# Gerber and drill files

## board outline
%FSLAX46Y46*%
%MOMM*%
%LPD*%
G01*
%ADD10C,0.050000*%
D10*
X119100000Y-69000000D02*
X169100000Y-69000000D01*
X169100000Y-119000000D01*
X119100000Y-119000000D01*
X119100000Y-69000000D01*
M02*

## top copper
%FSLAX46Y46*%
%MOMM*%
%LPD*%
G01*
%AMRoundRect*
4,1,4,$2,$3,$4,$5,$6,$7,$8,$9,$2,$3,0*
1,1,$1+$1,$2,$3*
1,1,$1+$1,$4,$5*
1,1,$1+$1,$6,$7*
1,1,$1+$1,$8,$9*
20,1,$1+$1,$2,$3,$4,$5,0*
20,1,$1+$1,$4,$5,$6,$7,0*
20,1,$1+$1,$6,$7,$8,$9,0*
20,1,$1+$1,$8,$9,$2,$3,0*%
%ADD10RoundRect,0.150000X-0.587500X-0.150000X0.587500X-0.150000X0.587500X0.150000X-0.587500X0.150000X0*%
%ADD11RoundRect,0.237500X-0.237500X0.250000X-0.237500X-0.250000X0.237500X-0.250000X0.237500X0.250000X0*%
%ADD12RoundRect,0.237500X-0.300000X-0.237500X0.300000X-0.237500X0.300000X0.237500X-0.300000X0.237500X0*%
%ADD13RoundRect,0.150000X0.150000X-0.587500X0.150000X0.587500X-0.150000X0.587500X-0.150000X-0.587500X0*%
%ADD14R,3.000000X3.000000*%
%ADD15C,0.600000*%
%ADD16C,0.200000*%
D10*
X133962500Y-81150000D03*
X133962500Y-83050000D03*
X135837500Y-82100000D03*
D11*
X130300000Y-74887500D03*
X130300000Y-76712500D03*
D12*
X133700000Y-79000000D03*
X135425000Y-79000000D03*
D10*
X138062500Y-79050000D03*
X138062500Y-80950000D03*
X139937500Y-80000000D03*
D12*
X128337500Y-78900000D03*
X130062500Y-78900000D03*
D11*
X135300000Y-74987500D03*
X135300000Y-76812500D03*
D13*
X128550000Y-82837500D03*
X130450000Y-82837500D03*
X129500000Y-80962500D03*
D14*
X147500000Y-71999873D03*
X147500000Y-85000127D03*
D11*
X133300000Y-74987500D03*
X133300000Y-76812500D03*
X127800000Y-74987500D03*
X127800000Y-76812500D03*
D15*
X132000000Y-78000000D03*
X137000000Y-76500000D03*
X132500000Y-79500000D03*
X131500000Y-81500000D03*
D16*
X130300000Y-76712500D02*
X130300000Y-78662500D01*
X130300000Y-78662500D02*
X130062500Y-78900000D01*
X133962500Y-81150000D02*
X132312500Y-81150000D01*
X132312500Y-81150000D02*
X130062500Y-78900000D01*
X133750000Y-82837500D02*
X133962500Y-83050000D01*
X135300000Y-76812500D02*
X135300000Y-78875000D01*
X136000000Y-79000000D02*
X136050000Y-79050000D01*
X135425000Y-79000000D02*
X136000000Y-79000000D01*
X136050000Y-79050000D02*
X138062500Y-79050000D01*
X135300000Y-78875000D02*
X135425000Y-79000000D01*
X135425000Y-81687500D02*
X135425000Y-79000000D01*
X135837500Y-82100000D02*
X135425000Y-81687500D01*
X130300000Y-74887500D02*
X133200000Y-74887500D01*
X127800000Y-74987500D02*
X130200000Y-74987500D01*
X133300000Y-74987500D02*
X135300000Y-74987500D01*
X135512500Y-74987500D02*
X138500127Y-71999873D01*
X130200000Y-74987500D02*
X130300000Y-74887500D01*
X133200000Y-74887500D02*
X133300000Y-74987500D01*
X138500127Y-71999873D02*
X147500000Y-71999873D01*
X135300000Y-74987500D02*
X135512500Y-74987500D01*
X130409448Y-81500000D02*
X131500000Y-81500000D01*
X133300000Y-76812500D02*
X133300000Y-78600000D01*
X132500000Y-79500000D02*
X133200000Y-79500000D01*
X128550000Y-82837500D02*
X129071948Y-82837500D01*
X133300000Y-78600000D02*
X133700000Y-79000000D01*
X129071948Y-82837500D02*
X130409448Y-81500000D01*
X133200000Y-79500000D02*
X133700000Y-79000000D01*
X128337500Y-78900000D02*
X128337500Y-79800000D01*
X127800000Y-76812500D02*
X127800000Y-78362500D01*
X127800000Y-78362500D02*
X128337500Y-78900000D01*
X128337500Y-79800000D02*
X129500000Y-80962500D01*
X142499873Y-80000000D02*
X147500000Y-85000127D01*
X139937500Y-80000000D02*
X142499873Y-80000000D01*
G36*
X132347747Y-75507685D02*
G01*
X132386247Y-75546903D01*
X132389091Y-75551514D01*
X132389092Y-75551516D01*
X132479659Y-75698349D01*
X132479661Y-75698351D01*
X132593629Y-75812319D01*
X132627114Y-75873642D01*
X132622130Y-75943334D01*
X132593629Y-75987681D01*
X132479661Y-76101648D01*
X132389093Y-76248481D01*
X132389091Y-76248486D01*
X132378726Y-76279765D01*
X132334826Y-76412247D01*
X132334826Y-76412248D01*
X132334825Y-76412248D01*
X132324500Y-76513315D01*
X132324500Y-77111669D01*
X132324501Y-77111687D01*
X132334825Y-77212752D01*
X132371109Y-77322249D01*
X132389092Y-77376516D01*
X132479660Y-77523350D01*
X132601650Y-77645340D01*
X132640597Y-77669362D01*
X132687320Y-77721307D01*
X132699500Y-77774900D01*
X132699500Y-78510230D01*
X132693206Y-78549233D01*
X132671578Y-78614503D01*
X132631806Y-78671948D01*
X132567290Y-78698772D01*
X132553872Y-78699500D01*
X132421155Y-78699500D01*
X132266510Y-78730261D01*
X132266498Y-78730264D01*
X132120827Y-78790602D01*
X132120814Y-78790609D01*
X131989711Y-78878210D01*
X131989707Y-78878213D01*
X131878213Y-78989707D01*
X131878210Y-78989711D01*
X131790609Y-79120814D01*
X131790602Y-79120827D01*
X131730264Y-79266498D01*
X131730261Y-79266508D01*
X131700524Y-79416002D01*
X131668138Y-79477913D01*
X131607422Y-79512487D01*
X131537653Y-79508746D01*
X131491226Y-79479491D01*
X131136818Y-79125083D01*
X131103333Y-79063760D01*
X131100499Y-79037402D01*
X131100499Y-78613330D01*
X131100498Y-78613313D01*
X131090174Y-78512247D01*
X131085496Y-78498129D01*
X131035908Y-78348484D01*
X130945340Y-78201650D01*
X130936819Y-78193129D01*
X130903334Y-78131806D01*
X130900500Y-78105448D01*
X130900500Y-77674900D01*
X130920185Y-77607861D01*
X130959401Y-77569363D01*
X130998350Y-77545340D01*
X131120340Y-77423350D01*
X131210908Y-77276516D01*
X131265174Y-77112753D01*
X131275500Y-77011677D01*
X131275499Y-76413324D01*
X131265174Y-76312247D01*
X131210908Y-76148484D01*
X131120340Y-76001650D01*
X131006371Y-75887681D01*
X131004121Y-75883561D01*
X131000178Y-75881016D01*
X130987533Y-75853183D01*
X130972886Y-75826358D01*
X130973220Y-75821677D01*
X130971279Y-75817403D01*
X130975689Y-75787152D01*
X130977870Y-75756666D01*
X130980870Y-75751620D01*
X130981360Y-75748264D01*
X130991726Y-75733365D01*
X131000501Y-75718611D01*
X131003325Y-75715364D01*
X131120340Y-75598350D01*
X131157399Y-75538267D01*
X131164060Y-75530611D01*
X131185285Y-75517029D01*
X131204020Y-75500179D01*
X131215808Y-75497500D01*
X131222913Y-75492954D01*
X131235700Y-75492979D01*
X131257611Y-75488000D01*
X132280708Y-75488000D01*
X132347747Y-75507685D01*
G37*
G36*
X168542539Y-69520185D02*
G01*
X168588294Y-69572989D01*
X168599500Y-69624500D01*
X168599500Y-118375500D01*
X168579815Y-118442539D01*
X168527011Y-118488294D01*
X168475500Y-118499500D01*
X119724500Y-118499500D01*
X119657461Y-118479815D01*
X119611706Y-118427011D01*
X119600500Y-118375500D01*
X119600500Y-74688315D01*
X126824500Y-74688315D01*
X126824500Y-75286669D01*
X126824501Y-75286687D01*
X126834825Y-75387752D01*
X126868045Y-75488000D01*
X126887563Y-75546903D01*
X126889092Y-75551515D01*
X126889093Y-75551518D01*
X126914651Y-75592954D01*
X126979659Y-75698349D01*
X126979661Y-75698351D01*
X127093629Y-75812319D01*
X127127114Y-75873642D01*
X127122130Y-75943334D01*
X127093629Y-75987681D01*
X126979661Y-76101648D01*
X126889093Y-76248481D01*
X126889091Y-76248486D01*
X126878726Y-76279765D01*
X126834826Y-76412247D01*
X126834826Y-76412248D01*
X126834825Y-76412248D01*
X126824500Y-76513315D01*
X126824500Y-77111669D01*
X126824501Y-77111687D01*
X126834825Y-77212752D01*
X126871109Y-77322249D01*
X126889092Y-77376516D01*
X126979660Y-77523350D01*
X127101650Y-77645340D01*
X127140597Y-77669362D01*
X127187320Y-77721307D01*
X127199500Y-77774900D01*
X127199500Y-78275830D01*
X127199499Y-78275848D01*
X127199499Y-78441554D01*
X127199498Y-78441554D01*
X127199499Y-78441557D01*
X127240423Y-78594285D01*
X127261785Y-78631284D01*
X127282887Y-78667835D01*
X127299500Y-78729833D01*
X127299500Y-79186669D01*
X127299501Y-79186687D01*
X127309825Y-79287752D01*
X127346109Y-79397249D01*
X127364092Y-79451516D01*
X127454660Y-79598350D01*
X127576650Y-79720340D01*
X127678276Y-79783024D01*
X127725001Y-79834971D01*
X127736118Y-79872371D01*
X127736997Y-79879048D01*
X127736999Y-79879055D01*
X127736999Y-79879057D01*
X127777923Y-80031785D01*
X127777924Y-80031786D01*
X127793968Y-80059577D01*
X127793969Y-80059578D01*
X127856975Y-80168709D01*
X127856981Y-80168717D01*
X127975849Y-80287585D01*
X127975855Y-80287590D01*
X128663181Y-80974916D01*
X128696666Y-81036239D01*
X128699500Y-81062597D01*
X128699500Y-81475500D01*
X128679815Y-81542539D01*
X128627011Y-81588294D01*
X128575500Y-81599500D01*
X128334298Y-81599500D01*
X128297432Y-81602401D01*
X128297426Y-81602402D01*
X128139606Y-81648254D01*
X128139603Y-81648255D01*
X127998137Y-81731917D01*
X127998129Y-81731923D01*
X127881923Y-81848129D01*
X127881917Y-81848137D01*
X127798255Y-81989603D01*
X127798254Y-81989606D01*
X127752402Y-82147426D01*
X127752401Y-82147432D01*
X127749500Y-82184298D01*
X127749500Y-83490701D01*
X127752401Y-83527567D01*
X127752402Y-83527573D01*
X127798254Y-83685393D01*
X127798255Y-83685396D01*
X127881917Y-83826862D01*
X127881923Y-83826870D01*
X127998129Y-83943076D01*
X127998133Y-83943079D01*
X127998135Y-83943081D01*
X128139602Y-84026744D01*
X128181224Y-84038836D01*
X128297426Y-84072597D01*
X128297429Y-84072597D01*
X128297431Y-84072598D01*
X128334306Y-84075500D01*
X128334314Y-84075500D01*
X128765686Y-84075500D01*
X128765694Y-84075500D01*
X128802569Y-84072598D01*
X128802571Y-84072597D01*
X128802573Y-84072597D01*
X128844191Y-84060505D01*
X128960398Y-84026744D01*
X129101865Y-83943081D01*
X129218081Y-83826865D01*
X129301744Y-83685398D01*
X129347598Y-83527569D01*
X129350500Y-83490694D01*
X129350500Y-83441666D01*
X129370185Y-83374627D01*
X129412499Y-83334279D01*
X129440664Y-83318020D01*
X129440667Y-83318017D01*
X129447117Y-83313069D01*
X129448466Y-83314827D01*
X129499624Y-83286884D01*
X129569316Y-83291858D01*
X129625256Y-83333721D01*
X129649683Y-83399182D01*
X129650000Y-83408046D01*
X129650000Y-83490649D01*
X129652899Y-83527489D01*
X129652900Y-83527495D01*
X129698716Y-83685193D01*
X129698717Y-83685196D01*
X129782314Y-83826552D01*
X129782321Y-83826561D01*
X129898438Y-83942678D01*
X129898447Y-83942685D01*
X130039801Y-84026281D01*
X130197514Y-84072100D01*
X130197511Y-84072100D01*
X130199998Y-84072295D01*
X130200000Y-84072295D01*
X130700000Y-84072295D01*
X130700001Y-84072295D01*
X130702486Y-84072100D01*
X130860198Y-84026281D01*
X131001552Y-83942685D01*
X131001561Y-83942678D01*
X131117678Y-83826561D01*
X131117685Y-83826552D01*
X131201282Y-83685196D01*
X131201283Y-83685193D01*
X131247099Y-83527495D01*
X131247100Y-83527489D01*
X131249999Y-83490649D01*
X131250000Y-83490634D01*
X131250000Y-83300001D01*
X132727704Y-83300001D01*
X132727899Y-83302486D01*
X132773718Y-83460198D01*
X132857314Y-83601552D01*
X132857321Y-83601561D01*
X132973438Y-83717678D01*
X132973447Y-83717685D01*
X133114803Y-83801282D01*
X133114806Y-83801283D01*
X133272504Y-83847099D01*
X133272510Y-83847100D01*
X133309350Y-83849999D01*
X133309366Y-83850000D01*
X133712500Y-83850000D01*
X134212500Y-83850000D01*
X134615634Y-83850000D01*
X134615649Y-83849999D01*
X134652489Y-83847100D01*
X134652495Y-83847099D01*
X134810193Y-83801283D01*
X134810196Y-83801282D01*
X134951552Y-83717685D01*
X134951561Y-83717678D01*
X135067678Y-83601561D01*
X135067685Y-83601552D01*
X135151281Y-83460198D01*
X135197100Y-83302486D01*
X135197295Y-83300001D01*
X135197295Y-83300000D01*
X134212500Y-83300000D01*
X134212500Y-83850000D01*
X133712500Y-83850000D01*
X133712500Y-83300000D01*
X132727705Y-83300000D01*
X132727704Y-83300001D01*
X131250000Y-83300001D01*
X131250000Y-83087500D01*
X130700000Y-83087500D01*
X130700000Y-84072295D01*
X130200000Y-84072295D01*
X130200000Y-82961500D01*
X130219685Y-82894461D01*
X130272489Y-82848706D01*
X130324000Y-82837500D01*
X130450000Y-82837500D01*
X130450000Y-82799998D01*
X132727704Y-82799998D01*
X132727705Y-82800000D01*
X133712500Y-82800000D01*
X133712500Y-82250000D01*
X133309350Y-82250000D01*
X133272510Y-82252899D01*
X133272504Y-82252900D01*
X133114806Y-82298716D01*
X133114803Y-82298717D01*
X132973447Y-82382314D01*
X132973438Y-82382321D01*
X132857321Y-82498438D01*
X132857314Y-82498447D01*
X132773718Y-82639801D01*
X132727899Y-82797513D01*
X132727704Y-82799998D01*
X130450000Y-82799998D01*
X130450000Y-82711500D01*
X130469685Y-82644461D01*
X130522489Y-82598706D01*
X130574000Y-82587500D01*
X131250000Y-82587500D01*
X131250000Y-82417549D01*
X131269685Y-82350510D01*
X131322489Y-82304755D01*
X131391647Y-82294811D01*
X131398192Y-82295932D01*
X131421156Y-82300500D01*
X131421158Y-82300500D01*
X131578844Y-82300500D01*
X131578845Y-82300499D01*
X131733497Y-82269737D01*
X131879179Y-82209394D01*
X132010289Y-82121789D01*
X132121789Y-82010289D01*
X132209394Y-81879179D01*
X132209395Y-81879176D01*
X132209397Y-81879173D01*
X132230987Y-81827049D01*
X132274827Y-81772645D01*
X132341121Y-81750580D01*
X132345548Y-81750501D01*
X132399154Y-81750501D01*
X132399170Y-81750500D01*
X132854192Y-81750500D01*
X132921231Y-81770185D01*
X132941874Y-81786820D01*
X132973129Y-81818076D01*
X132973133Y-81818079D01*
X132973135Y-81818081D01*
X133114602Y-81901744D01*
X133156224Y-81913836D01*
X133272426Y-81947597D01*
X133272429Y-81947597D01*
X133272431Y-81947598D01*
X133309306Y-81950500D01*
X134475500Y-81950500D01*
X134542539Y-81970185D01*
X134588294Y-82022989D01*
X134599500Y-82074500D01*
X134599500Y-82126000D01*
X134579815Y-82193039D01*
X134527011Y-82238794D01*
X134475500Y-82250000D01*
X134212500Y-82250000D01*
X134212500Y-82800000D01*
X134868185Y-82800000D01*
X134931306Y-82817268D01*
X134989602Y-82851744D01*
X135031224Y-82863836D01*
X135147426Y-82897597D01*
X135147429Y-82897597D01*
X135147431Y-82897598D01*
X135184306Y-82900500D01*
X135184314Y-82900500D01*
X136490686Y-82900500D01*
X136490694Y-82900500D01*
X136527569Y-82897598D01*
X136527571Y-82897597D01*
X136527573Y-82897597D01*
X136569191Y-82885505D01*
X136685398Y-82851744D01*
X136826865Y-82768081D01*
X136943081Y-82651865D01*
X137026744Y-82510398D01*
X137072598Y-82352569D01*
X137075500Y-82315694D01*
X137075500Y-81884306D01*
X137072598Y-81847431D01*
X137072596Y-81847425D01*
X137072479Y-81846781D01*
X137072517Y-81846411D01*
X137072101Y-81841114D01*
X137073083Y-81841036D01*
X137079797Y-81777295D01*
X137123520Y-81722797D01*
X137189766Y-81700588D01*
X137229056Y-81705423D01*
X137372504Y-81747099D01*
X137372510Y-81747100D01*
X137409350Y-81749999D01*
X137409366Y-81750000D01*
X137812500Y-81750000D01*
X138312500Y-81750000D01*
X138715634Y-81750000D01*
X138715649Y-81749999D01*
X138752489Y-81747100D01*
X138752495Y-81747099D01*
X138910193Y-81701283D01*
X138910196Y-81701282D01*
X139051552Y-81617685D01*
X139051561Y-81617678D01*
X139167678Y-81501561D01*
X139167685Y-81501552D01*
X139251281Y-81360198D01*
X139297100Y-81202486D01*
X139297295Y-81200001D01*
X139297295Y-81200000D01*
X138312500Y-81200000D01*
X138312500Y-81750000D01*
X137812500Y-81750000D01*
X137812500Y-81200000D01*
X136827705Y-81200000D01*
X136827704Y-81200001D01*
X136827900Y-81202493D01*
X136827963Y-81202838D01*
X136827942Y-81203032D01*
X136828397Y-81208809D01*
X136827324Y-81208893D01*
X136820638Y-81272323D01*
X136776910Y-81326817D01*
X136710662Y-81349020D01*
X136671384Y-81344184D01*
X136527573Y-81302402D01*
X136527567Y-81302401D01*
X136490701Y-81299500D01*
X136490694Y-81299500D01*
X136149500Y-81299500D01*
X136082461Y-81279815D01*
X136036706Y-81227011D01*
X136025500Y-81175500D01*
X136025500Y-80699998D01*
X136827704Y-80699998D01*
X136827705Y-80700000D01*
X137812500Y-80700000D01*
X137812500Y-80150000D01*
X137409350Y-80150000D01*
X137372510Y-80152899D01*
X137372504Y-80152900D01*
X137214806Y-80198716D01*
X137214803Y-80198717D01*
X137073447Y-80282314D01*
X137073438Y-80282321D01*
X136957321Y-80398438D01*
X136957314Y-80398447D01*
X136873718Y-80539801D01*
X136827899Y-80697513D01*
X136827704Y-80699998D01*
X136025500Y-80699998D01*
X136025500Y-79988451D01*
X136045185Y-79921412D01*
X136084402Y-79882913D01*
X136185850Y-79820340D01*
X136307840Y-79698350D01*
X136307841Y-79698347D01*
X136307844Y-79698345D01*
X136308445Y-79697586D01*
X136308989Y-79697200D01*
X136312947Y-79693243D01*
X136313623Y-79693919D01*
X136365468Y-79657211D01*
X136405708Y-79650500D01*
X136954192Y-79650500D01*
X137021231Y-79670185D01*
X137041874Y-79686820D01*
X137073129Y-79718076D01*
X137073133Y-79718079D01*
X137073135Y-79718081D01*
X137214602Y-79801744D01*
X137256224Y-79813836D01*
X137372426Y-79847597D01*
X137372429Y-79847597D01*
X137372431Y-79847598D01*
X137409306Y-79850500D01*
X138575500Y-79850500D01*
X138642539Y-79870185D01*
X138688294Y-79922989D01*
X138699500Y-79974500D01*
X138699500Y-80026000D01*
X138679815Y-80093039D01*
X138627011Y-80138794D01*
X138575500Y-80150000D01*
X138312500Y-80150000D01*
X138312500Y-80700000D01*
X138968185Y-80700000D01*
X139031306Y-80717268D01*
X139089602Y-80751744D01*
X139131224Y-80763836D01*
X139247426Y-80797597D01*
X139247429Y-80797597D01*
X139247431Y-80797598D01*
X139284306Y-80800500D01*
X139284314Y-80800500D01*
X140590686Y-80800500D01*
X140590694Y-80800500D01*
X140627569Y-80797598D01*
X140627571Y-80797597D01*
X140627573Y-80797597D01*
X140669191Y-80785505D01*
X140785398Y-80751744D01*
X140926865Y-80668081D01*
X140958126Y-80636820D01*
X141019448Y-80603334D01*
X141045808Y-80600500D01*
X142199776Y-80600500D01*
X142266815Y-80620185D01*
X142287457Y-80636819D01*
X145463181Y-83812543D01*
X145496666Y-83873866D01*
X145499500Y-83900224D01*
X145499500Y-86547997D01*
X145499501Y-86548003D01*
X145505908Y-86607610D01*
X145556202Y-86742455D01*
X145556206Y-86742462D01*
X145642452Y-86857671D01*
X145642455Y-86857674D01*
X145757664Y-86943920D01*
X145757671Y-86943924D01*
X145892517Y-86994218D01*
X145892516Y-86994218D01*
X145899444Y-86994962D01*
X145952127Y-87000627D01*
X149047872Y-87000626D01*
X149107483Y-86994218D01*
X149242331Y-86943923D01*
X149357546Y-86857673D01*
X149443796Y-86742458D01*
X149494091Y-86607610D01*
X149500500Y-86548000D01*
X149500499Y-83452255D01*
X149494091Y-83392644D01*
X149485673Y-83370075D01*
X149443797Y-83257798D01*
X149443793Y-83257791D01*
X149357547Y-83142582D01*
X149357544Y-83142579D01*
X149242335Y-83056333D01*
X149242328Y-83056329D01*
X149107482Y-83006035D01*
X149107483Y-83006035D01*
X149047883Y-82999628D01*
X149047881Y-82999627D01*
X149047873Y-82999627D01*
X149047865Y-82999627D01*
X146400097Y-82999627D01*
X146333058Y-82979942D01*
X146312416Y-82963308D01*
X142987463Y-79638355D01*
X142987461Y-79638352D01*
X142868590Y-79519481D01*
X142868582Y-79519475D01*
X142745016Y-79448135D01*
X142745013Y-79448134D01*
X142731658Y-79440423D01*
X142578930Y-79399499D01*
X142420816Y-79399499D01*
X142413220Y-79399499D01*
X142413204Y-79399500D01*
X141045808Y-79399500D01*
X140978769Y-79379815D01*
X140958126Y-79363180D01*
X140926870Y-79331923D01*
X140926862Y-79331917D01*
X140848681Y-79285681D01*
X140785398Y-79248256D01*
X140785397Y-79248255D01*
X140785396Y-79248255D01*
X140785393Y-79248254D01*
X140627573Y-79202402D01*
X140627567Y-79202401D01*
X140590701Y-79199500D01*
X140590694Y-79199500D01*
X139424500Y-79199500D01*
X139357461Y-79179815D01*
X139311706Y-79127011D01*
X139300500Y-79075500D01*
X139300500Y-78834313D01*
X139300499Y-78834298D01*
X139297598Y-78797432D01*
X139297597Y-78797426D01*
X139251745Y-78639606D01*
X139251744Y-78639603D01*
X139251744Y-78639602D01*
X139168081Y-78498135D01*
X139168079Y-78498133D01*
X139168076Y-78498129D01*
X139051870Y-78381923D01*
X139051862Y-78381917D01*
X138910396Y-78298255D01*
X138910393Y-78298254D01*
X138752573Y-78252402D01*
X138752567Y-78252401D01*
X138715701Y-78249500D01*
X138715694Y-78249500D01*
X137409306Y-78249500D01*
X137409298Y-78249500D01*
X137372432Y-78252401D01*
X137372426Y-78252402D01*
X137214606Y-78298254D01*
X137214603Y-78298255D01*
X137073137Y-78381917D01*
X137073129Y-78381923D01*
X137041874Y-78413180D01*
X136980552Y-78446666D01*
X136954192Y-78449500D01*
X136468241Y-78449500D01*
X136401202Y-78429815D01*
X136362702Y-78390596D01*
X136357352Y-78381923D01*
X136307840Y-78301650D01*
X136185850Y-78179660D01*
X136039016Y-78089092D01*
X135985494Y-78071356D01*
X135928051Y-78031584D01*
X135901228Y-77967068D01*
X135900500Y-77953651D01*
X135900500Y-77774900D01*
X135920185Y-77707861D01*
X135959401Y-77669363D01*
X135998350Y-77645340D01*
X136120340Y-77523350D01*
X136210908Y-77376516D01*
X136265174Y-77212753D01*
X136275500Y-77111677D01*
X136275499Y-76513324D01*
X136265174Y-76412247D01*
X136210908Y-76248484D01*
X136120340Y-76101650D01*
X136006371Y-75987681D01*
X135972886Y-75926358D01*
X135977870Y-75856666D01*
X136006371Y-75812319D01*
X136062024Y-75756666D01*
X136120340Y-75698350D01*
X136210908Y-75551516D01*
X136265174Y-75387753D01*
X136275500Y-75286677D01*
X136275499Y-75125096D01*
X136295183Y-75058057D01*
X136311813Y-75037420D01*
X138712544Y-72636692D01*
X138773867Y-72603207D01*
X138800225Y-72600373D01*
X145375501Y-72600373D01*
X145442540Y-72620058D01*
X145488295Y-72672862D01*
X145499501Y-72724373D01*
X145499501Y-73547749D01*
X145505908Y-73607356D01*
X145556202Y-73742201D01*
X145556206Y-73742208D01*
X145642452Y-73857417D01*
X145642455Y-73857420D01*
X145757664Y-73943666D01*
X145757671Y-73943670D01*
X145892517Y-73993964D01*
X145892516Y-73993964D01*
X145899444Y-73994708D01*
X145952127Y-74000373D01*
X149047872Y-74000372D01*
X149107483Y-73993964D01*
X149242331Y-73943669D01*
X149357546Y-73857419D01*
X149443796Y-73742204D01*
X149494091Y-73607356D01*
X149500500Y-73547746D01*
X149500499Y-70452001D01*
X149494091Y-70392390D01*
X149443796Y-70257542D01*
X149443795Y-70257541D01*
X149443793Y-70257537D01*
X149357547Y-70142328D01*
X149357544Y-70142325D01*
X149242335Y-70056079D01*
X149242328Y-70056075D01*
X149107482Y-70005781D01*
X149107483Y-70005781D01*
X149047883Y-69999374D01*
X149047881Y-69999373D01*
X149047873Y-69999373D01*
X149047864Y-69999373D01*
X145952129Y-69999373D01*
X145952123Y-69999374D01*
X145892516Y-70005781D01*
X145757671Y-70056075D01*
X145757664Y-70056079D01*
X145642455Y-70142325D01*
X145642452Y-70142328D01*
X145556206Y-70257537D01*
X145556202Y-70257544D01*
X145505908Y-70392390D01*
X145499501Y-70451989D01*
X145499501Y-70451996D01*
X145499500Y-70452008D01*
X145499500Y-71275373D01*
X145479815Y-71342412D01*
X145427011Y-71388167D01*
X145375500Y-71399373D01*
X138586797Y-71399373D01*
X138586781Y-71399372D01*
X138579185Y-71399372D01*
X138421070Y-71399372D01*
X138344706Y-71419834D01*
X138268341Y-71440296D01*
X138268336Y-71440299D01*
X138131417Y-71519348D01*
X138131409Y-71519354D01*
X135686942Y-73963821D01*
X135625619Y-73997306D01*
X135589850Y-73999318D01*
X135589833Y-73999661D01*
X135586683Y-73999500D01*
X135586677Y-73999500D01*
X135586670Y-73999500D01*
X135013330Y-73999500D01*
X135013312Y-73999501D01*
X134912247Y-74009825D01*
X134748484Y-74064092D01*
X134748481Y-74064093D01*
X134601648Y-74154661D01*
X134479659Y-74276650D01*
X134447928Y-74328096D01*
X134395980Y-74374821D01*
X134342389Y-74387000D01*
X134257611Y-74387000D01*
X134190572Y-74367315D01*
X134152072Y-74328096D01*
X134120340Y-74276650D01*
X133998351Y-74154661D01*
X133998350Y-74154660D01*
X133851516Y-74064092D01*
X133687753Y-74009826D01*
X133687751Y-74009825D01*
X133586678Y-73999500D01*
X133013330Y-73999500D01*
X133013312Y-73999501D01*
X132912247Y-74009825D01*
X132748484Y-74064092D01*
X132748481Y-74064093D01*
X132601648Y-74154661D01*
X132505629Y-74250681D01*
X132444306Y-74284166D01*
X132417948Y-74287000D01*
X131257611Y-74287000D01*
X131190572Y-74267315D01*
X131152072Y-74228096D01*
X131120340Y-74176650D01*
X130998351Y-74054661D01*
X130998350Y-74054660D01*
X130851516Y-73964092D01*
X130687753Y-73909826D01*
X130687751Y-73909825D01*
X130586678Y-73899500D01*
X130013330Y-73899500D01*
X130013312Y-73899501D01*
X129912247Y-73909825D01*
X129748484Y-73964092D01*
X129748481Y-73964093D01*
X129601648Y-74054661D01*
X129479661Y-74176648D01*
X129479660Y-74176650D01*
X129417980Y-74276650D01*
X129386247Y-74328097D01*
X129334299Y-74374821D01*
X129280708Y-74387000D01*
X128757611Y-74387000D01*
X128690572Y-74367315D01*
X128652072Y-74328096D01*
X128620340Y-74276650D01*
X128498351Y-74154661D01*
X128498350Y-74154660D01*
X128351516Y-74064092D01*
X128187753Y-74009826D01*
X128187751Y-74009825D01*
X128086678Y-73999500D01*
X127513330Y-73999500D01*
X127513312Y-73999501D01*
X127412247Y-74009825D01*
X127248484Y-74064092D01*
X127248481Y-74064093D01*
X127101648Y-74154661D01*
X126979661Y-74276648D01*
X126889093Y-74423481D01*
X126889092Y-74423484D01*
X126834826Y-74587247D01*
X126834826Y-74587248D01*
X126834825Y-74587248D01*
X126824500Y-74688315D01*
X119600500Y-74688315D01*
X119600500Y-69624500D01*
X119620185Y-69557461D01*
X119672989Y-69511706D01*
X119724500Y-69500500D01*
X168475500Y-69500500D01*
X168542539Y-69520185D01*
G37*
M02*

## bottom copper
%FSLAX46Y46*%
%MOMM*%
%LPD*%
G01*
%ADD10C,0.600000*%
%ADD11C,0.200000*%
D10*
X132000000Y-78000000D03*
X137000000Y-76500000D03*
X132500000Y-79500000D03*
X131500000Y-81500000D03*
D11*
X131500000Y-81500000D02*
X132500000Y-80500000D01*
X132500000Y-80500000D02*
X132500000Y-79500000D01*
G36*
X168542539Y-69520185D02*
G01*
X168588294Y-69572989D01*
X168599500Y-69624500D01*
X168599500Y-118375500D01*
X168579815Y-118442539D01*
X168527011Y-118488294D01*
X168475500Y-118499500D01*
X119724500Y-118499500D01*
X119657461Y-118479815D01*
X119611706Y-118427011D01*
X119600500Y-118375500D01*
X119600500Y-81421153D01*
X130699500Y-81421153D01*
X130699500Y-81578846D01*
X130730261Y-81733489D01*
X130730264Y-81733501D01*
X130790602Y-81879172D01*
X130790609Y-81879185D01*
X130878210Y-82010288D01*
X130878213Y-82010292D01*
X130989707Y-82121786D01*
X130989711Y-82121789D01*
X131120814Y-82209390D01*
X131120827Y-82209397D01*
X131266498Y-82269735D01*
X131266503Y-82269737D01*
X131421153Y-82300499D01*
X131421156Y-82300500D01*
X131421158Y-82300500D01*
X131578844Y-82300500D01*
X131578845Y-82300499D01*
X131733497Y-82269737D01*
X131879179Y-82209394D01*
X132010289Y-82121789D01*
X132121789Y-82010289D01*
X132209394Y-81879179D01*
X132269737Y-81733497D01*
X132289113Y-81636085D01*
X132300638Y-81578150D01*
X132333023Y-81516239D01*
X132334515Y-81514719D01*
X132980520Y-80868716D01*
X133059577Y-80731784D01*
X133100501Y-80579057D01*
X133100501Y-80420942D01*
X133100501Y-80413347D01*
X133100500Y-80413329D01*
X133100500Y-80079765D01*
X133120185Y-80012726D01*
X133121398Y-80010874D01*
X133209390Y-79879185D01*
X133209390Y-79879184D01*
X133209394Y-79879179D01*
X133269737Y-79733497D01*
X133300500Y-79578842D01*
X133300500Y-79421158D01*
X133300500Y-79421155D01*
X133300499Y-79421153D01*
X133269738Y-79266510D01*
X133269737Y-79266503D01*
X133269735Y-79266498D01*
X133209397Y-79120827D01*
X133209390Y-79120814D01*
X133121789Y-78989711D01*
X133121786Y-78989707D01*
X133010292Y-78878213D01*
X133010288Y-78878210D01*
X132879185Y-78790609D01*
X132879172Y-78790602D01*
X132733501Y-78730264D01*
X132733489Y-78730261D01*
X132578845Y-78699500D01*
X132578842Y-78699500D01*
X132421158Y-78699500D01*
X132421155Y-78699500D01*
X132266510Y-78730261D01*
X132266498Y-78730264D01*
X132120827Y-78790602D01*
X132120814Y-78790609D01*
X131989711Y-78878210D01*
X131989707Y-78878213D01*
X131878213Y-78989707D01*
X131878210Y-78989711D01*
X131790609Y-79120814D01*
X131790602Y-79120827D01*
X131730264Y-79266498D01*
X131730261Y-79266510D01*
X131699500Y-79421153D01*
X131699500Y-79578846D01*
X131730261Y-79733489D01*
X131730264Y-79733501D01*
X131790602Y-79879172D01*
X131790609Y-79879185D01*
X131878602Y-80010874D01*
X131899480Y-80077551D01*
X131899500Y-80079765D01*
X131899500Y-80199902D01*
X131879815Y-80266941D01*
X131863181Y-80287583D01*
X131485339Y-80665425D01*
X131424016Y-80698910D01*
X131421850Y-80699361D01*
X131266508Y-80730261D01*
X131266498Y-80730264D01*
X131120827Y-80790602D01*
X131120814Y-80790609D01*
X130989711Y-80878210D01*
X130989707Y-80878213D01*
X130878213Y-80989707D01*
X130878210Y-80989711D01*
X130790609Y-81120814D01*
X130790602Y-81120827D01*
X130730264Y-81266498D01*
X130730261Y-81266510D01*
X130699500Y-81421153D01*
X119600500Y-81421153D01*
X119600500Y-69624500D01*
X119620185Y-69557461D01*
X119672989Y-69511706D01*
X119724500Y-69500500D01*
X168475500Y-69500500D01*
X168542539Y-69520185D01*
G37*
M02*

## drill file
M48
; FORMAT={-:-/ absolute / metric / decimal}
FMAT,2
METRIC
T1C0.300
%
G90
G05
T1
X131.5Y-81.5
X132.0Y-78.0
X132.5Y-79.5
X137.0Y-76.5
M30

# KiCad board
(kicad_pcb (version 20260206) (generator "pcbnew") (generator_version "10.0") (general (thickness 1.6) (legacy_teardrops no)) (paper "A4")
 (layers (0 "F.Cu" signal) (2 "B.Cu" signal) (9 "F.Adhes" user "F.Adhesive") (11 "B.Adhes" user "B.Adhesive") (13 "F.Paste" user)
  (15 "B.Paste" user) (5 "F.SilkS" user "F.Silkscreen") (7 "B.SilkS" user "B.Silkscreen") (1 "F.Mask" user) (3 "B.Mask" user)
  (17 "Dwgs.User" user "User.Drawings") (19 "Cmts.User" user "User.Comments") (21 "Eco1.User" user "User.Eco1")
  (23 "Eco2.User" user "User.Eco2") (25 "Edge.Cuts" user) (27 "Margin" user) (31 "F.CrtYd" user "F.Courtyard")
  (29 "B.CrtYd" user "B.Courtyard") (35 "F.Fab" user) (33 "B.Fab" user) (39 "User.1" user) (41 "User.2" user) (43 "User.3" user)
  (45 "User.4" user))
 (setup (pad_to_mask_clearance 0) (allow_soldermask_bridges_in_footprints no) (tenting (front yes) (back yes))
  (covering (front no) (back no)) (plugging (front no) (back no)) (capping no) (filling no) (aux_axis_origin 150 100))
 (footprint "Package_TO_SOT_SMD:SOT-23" (layer "F.Cu") (at 134.9 82.1)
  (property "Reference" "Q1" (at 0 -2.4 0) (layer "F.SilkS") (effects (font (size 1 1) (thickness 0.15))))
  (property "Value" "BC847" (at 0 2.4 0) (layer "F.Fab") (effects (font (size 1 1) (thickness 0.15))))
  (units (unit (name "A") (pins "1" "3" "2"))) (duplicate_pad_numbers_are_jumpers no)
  (pad "1" smd roundrect (at -0.9375 -0.95) (size 1.475 0.6) (layers "F.Cu" "F.Mask" "F.Paste") (roundrect_rratio 0.25) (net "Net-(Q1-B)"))
  (pad "2" smd roundrect (at -0.9375 0.95) (size 1.475 0.6) (layers "F.Cu" "F.Mask" "F.Paste") (roundrect_rratio 0.25) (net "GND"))
  (pad "3" smd roundrect (at 0.9375 0) (size 1.475 0.6) (layers "F.Cu" "F.Mask" "F.Paste") (roundrect_rratio 0.25) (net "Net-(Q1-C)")))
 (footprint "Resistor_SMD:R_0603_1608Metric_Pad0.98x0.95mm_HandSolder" (layer "F.Cu") (at 130.3 75.8 -90)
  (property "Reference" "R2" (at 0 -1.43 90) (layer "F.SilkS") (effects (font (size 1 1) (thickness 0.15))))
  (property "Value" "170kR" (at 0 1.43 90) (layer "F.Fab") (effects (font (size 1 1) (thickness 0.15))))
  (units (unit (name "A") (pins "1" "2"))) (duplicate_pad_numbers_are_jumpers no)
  (pad "1" smd roundrect (at -0.9125 0 270) (size 0.975 0.95) (layers "F.Cu" "F.Mask" "F.Paste") (roundrect_rratio 0.25) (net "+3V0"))
  (pad "2" smd roundrect (at 0.9125 0 270) (size 0.975 0.95) (layers "F.Cu" "F.Mask" "F.Paste") (roundrect_rratio 0.25) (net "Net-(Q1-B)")))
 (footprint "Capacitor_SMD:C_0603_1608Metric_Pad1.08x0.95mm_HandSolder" (layer "F.Cu") (at 134.5625 79)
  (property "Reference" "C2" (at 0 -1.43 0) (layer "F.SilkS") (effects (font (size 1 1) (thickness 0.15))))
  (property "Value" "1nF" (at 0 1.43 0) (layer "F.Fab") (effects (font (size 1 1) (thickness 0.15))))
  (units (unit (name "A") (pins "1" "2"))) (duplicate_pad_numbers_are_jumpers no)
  (pad "1" smd roundrect (at -0.8625 0) (size 1.075 0.95) (layers "F.Cu" "F.Mask" "F.Paste") (roundrect_rratio 0.25) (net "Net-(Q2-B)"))
  (pad "2" smd roundrect (at 0.8625 0) (size 1.075 0.95) (layers "F.Cu" "F.Mask" "F.Paste") (roundrect_rratio 0.25) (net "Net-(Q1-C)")))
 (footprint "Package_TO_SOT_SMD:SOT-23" (layer "F.Cu") (at 139 80)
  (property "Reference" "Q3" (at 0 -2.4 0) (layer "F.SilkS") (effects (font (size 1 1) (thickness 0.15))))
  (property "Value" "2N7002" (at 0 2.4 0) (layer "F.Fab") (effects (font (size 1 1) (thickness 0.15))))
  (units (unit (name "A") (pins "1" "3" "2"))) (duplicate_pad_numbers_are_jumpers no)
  (pad "1" smd roundrect (at -0.9375 -0.95) (size 1.475 0.6) (layers "F.Cu" "F.Mask" "F.Paste") (roundrect_rratio 0.25) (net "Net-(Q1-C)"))
  (pad "2" smd roundrect (at -0.9375 0.95) (size 1.475 0.6) (layers "F.Cu" "F.Mask" "F.Paste") (roundrect_rratio 0.25) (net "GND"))
  (pad "3" smd roundrect (at 0.9375 0) (size 1.475 0.6) (layers "F.Cu" "F.Mask" "F.Paste") (roundrect_rratio 0.25) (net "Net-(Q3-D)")))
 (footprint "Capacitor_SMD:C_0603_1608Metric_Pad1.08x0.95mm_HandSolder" (layer "F.Cu") (at 129.2 78.9)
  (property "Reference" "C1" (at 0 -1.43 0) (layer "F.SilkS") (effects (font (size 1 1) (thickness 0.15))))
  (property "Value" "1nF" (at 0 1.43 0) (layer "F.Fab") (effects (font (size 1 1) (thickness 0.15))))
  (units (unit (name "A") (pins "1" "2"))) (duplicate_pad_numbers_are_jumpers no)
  (pad "1" smd roundrect (at -0.8625 0) (size 1.075 0.95) (layers "F.Cu" "F.Mask" "F.Paste") (roundrect_rratio 0.25) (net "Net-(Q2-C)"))
  (pad "2" smd roundrect (at 0.8625 0) (size 1.075 0.95) (layers "F.Cu" "F.Mask" "F.Paste") (roundrect_rratio 0.25) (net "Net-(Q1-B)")))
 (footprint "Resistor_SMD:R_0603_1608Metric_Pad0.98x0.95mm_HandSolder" (layer "F.Cu") (at 135.3 75.9 -90)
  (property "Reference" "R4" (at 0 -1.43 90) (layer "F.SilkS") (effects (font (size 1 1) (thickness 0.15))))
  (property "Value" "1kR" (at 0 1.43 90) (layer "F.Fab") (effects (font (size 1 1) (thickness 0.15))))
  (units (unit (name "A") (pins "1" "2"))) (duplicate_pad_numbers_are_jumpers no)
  (pad "1" smd roundrect (at -0.9125 0 270) (size 0.975 0.95) (layers "F.Cu" "F.Mask" "F.Paste") (roundrect_rratio 0.25) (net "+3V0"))
  (pad "2" smd roundrect (at 0.9125 0 270) (size 0.975 0.95) (layers "F.Cu" "F.Mask" "F.Paste") (roundrect_rratio 0.25) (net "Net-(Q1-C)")))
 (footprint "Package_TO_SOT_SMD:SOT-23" (layer "F.Cu") (at 129.5 81.9 90)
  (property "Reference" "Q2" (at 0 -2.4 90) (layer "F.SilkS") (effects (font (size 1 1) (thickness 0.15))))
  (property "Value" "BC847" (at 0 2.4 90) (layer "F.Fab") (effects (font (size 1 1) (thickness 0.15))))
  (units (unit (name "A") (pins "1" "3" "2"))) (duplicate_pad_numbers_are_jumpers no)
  (pad "1" smd roundrect (at -0.9375 -0.95 90) (size 1.475 0.6) (layers "F.Cu" "F.Mask" "F.Paste") (roundrect_rratio 0.25)
   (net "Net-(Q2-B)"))
  (pad "2" smd roundrect (at -0.9375 0.95 90) (size 1.475 0.6) (layers "F.Cu" "F.Mask" "F.Paste") (roundrect_rratio 0.25) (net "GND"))
  (pad "3" smd roundrect (at 0.9375 0 90) (size 1.475 0.6) (layers "F.Cu" "F.Mask" "F.Paste") (roundrect_rratio 0.25) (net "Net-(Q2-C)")))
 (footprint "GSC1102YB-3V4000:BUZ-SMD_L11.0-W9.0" (layer "F.Cu") (at 147.5 78.5 -90)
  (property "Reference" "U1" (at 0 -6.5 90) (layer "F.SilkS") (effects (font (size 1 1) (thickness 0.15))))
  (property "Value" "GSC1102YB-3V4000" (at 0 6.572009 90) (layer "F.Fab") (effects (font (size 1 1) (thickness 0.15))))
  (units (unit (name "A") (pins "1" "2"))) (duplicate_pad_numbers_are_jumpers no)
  (pad "1" smd rect (at -6.500127 0) (size 3 3) (layers "F.Cu" "F.Mask" "F.Paste") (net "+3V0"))
  (pad "2" smd rect (at 6.500127 0) (size 3 3) (layers "F.Cu" "F.Mask" "F.Paste") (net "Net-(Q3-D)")))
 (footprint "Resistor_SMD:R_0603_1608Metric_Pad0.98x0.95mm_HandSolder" (layer "F.Cu") (at 133.3 75.9 -90)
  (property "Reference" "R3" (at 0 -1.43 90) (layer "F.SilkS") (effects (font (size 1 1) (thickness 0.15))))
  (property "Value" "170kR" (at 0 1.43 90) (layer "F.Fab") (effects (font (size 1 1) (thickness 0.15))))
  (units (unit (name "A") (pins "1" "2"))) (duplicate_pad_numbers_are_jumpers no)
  (pad "1" smd roundrect (at -0.9125 0 270) (size 0.975 0.95) (layers "F.Cu" "F.Mask" "F.Paste") (roundrect_rratio 0.25) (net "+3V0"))
  (pad "2" smd roundrect (at 0.9125 0 270) (size 0.975 0.95) (layers "F.Cu" "F.Mask" "F.Paste") (roundrect_rratio 0.25) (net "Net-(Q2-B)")))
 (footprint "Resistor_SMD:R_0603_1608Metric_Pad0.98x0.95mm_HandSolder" (layer "F.Cu") (at 127.8 75.9 -90)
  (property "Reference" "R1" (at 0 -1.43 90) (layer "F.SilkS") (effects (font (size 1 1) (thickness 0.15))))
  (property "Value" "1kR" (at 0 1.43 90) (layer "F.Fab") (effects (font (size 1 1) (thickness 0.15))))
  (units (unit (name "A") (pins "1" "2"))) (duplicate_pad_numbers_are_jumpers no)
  (pad "1" smd roundrect (at -0.9125 0 270) (size 0.975 0.95) (layers "F.Cu" "F.Mask" "F.Paste") (roundrect_rratio 0.25) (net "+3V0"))
  (pad "2" smd roundrect (at 0.9125 0 270) (size 0.975 0.95) (layers "F.Cu" "F.Mask" "F.Paste") (roundrect_rratio 0.25) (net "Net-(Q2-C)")))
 (gr_rect (start 119.1 69) (end 169.1 119) (stroke (width 0.05) (type solid)) (fill no) (layer "Edge.Cuts"))
 (segment (start 130.3 76.7125) (end 130.3 78.6625) (width 0.2) (layer "F.Cu") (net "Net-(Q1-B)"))
 (segment (start 130.3 78.6625) (end 130.0625 78.9) (width 0.2) (layer "F.Cu") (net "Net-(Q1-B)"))
 (segment (start 133.9625 81.15) (end 132.3125 81.15) (width 0.2) (layer "F.Cu") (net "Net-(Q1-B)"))
 (segment (start 132.3125 81.15) (end 130.0625 78.9) (width 0.2) (layer "F.Cu") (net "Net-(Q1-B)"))
 (segment (start 133.75 82.8375) (end 133.9625 83.05) (width 0.2) (layer "F.Cu") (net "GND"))
 (via (at 132 78) (size 0.6) (drill 0.3) (layers "F.Cu" "B.Cu") (free yes) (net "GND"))
 (via (at 137 76.5) (size 0.6) (drill 0.3) (layers "F.Cu" "B.Cu") (free yes) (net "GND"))
 (segment (start 135.3 76.8125) (end 135.3 78.875) (width 0.2) (layer "F.Cu") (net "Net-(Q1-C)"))
 (segment (start 136 79) (end 136.05 79.05) (width 0.2) (layer "F.Cu") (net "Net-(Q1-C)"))
 (segment (start 135.425 79) (end 136 79) (width 0.2) (layer "F.Cu") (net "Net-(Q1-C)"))
 (segment (start 136.05 79.05) (end 138.0625 79.05) (width 0.2) (layer "F.Cu") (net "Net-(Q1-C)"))
 (segment (start 135.3 78.875) (end 135.425 79) (width 0.2) (layer "F.Cu") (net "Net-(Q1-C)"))
 (segment (start 135.425 81.6875) (end 135.425 79) (width 0.2) (layer "F.Cu") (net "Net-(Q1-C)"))
 (segment (start 135.8375 82.1) (end 135.425 81.6875) (width 0.2) (layer "F.Cu") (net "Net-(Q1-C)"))
 (segment (start 130.3 74.8875) (end 133.2 74.8875) (width 0.2) (layer "F.Cu") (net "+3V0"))
 (segment (start 127.8 74.9875) (end 130.2 74.9875) (width 0.2) (layer "F.Cu") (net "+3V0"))
 (segment (start 133.3 74.9875) (end 135.3 74.9875) (width 0.2) (layer "F.Cu") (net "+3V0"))
 (segment (start 135.5125 74.9875) (end 138.500127 71.999873) (width 0.2) (layer "F.Cu") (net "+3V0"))
 (segment (start 130.2 74.9875) (end 130.3 74.8875) (width 0.2) (layer "F.Cu") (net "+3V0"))
 (segment (start 133.2 74.8875) (end 133.3 74.9875) (width 0.2) (layer "F.Cu") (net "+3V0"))
 (segment (start 138.500127 71.999873) (end 147.5 71.999873) (width 0.2) (layer "F.Cu") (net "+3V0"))
 (segment (start 135.3 74.9875) (end 135.5125 74.9875) (width 0.2) (layer "F.Cu") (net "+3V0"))
 (segment (start 130.409448 81.5) (end 131.5 81.5) (width 0.2) (layer "F.Cu") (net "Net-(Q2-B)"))
 (segment (start 133.3 76.8125) (end 133.3 78.6) (width 0.2) (layer "F.Cu") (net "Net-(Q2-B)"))
 (segment (start 132.5 79.5) (end 133.2 79.5) (width 0.2) (layer "F.Cu") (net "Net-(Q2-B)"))
 (segment (start 128.55 82.8375) (end 129.071948 82.8375) (width 0.2) (layer "F.Cu") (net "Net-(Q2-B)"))
 (segment (start 133.3 78.6) (end 133.7 79) (width 0.2) (layer "F.Cu") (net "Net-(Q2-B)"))
 (segment (start 129.071948 82.8375) (end 130.409448 81.5) (width 0.2) (layer "F.Cu") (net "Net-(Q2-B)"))
 (segment (start 133.2 79.5) (end 133.7 79) (width 0.2) (layer "F.Cu") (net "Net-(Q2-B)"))
 (via (at 132.5 79.5) (size 0.6) (drill 0.3) (layers "F.Cu" "B.Cu") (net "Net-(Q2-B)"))
 (via (at 131.5 81.5) (size 0.6) (drill 0.3) (layers "F.Cu" "B.Cu") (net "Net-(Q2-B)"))
 (segment (start 131.5 81.5) (end 132.5 80.5) (width 0.2) (layer "B.Cu") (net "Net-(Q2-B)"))
 (segment (start 132.5 80.5) (end 132.5 79.5) (width 0.2) (layer "B.Cu") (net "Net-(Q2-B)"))
 (segment (start 128.3375 78.9) (end 128.3375 79.8) (width 0.2) (layer "F.Cu") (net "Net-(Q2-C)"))
 (segment (start 127.8 76.8125) (end 127.8 78.3625) (width 0.2) (layer "F.Cu") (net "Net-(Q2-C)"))
 (segment (start 127.8 78.3625) (end 128.3375 78.9) (width 0.2) (layer "F.Cu") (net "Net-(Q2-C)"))
 (segment (start 128.3375 79.8) (end 129.5 80.9625) (width 0.2) (layer "F.Cu") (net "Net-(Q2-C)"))
 (segment (start 142.499873 80) (end 147.5 85.000127) (width 0.2) (layer "F.Cu") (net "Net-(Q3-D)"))
 (segment (start 139.9375 80) (end 142.499873 80) (width 0.2) (layer "F.Cu") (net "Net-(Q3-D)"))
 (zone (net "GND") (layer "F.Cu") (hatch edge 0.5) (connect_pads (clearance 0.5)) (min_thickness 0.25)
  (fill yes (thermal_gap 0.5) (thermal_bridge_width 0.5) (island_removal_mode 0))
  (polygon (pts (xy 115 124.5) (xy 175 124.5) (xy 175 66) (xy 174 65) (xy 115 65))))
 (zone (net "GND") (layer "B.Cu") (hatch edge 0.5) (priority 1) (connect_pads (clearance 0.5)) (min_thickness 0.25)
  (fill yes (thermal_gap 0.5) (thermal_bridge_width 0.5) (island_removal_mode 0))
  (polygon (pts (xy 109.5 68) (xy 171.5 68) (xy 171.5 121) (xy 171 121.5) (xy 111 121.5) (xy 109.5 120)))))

